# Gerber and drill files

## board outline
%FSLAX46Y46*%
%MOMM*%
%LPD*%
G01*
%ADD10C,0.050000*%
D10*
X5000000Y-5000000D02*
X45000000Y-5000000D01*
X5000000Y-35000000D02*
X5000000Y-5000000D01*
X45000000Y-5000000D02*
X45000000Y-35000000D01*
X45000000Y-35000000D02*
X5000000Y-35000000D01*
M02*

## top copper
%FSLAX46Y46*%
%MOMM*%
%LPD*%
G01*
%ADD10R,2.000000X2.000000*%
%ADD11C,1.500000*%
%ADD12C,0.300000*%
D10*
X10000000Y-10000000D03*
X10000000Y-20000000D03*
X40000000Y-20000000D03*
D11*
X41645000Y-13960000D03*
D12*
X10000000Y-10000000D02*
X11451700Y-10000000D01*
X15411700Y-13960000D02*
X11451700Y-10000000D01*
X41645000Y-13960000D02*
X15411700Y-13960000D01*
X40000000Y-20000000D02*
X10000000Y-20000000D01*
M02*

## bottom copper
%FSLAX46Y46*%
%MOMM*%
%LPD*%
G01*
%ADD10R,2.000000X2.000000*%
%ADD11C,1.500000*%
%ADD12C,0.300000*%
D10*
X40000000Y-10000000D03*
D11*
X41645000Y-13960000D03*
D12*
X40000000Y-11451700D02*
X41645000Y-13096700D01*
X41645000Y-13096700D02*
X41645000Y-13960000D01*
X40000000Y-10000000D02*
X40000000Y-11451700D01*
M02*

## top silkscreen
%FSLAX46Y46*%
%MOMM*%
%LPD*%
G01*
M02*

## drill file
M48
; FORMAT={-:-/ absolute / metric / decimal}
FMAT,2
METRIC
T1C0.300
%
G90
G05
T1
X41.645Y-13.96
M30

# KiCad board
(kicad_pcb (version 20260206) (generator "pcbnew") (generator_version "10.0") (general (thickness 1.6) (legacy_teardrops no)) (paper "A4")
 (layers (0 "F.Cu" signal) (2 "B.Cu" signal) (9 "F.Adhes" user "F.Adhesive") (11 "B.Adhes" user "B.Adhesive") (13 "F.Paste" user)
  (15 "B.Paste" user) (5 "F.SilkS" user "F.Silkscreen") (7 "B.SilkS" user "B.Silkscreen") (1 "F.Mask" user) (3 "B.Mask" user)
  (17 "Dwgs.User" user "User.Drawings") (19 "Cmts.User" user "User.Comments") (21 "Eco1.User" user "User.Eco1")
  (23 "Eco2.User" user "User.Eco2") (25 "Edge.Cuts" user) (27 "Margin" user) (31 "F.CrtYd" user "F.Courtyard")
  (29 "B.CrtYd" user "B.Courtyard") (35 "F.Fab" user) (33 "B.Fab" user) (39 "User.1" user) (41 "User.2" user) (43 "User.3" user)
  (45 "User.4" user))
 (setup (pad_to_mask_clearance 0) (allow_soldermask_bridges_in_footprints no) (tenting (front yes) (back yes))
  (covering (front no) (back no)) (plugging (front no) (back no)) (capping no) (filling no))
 (gr_line (start 5 5) (end 45 5) (stroke (width 0.05) (type default)) (layer "Edge.Cuts"))
 (gr_line (start 5 35) (end 5 5) (stroke (width 0.05) (type default)) (layer "Edge.Cuts"))
 (gr_line (start 45 5) (end 45 35) (stroke (width 0.05) (type default)) (layer "Edge.Cuts"))
 (gr_line (start 45 35) (end 5 35) (stroke (width 0.05) (type default)) (layer "Edge.Cuts"))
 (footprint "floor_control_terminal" (layer "F.Cu") (at 10 10)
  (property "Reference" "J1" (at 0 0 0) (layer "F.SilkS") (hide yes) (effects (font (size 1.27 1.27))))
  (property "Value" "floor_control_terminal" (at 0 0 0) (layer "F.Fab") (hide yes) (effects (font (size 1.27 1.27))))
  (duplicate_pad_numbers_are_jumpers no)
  (pad "1" smd rect (at 0 0) (size 2 2) (layers "F.Cu" "F.Paste" "F.Mask") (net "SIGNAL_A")))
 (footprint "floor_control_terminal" (layer "B.Cu") (at 40 10)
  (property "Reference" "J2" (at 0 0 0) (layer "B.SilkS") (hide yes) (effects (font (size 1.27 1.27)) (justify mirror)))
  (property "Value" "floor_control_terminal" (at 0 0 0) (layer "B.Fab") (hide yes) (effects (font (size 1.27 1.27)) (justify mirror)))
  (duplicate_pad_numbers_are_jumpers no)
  (pad "1" smd rect (at 0 0) (size 2 2) (layers "B.Cu" "B.Paste" "B.Mask") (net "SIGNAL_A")))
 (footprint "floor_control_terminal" (layer "F.Cu") (at 10 20)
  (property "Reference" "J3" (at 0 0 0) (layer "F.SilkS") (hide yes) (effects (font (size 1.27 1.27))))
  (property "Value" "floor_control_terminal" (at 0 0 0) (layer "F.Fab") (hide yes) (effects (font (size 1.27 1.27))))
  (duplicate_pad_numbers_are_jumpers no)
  (pad "1" smd rect (at 0 0) (size 2 2) (layers "F.Cu" "F.Paste" "F.Mask") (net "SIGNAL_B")))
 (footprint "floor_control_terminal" (layer "F.Cu") (at 40 20)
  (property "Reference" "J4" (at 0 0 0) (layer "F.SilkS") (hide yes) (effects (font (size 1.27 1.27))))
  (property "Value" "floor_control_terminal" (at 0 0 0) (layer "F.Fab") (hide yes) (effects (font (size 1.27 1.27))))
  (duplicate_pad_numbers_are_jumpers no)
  (pad "1" smd rect (at 0 0) (size 2 2) (layers "F.Cu" "F.Paste" "F.Mask") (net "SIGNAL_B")))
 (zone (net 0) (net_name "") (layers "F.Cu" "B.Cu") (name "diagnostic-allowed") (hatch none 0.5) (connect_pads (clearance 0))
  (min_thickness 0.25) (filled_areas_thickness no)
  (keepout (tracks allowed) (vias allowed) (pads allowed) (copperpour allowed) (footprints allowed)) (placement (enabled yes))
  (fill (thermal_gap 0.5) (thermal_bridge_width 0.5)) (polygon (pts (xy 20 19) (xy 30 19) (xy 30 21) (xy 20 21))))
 (segment (start 10 10) (end 11.4517 10) (width 0.3) (layer "F.Cu") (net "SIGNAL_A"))
 (segment (start 15.4117 13.96) (end 11.4517 10) (width 0.3) (layer "F.Cu") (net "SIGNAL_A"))
 (segment (start 41.645 13.96) (end 15.4117 13.96) (width 0.3) (layer "F.Cu") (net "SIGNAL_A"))
 (via (at 41.645 13.96) (size 1.5) (drill 0.3) (layers "F.Cu" "B.Cu") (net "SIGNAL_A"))
 (segment (start 40 11.4517) (end 41.645 13.0967) (width 0.3) (layer "B.Cu") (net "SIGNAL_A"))
 (segment (start 41.645 13.0967) (end 41.645 13.96) (width 0.3) (layer "B.Cu") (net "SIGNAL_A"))
 (segment (start 40 10) (end 40 11.4517) (width 0.3) (layer "B.Cu") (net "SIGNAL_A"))
 (segment (start 40 20) (end 10 20) (width 0.3) (layer "F.Cu") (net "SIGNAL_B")))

